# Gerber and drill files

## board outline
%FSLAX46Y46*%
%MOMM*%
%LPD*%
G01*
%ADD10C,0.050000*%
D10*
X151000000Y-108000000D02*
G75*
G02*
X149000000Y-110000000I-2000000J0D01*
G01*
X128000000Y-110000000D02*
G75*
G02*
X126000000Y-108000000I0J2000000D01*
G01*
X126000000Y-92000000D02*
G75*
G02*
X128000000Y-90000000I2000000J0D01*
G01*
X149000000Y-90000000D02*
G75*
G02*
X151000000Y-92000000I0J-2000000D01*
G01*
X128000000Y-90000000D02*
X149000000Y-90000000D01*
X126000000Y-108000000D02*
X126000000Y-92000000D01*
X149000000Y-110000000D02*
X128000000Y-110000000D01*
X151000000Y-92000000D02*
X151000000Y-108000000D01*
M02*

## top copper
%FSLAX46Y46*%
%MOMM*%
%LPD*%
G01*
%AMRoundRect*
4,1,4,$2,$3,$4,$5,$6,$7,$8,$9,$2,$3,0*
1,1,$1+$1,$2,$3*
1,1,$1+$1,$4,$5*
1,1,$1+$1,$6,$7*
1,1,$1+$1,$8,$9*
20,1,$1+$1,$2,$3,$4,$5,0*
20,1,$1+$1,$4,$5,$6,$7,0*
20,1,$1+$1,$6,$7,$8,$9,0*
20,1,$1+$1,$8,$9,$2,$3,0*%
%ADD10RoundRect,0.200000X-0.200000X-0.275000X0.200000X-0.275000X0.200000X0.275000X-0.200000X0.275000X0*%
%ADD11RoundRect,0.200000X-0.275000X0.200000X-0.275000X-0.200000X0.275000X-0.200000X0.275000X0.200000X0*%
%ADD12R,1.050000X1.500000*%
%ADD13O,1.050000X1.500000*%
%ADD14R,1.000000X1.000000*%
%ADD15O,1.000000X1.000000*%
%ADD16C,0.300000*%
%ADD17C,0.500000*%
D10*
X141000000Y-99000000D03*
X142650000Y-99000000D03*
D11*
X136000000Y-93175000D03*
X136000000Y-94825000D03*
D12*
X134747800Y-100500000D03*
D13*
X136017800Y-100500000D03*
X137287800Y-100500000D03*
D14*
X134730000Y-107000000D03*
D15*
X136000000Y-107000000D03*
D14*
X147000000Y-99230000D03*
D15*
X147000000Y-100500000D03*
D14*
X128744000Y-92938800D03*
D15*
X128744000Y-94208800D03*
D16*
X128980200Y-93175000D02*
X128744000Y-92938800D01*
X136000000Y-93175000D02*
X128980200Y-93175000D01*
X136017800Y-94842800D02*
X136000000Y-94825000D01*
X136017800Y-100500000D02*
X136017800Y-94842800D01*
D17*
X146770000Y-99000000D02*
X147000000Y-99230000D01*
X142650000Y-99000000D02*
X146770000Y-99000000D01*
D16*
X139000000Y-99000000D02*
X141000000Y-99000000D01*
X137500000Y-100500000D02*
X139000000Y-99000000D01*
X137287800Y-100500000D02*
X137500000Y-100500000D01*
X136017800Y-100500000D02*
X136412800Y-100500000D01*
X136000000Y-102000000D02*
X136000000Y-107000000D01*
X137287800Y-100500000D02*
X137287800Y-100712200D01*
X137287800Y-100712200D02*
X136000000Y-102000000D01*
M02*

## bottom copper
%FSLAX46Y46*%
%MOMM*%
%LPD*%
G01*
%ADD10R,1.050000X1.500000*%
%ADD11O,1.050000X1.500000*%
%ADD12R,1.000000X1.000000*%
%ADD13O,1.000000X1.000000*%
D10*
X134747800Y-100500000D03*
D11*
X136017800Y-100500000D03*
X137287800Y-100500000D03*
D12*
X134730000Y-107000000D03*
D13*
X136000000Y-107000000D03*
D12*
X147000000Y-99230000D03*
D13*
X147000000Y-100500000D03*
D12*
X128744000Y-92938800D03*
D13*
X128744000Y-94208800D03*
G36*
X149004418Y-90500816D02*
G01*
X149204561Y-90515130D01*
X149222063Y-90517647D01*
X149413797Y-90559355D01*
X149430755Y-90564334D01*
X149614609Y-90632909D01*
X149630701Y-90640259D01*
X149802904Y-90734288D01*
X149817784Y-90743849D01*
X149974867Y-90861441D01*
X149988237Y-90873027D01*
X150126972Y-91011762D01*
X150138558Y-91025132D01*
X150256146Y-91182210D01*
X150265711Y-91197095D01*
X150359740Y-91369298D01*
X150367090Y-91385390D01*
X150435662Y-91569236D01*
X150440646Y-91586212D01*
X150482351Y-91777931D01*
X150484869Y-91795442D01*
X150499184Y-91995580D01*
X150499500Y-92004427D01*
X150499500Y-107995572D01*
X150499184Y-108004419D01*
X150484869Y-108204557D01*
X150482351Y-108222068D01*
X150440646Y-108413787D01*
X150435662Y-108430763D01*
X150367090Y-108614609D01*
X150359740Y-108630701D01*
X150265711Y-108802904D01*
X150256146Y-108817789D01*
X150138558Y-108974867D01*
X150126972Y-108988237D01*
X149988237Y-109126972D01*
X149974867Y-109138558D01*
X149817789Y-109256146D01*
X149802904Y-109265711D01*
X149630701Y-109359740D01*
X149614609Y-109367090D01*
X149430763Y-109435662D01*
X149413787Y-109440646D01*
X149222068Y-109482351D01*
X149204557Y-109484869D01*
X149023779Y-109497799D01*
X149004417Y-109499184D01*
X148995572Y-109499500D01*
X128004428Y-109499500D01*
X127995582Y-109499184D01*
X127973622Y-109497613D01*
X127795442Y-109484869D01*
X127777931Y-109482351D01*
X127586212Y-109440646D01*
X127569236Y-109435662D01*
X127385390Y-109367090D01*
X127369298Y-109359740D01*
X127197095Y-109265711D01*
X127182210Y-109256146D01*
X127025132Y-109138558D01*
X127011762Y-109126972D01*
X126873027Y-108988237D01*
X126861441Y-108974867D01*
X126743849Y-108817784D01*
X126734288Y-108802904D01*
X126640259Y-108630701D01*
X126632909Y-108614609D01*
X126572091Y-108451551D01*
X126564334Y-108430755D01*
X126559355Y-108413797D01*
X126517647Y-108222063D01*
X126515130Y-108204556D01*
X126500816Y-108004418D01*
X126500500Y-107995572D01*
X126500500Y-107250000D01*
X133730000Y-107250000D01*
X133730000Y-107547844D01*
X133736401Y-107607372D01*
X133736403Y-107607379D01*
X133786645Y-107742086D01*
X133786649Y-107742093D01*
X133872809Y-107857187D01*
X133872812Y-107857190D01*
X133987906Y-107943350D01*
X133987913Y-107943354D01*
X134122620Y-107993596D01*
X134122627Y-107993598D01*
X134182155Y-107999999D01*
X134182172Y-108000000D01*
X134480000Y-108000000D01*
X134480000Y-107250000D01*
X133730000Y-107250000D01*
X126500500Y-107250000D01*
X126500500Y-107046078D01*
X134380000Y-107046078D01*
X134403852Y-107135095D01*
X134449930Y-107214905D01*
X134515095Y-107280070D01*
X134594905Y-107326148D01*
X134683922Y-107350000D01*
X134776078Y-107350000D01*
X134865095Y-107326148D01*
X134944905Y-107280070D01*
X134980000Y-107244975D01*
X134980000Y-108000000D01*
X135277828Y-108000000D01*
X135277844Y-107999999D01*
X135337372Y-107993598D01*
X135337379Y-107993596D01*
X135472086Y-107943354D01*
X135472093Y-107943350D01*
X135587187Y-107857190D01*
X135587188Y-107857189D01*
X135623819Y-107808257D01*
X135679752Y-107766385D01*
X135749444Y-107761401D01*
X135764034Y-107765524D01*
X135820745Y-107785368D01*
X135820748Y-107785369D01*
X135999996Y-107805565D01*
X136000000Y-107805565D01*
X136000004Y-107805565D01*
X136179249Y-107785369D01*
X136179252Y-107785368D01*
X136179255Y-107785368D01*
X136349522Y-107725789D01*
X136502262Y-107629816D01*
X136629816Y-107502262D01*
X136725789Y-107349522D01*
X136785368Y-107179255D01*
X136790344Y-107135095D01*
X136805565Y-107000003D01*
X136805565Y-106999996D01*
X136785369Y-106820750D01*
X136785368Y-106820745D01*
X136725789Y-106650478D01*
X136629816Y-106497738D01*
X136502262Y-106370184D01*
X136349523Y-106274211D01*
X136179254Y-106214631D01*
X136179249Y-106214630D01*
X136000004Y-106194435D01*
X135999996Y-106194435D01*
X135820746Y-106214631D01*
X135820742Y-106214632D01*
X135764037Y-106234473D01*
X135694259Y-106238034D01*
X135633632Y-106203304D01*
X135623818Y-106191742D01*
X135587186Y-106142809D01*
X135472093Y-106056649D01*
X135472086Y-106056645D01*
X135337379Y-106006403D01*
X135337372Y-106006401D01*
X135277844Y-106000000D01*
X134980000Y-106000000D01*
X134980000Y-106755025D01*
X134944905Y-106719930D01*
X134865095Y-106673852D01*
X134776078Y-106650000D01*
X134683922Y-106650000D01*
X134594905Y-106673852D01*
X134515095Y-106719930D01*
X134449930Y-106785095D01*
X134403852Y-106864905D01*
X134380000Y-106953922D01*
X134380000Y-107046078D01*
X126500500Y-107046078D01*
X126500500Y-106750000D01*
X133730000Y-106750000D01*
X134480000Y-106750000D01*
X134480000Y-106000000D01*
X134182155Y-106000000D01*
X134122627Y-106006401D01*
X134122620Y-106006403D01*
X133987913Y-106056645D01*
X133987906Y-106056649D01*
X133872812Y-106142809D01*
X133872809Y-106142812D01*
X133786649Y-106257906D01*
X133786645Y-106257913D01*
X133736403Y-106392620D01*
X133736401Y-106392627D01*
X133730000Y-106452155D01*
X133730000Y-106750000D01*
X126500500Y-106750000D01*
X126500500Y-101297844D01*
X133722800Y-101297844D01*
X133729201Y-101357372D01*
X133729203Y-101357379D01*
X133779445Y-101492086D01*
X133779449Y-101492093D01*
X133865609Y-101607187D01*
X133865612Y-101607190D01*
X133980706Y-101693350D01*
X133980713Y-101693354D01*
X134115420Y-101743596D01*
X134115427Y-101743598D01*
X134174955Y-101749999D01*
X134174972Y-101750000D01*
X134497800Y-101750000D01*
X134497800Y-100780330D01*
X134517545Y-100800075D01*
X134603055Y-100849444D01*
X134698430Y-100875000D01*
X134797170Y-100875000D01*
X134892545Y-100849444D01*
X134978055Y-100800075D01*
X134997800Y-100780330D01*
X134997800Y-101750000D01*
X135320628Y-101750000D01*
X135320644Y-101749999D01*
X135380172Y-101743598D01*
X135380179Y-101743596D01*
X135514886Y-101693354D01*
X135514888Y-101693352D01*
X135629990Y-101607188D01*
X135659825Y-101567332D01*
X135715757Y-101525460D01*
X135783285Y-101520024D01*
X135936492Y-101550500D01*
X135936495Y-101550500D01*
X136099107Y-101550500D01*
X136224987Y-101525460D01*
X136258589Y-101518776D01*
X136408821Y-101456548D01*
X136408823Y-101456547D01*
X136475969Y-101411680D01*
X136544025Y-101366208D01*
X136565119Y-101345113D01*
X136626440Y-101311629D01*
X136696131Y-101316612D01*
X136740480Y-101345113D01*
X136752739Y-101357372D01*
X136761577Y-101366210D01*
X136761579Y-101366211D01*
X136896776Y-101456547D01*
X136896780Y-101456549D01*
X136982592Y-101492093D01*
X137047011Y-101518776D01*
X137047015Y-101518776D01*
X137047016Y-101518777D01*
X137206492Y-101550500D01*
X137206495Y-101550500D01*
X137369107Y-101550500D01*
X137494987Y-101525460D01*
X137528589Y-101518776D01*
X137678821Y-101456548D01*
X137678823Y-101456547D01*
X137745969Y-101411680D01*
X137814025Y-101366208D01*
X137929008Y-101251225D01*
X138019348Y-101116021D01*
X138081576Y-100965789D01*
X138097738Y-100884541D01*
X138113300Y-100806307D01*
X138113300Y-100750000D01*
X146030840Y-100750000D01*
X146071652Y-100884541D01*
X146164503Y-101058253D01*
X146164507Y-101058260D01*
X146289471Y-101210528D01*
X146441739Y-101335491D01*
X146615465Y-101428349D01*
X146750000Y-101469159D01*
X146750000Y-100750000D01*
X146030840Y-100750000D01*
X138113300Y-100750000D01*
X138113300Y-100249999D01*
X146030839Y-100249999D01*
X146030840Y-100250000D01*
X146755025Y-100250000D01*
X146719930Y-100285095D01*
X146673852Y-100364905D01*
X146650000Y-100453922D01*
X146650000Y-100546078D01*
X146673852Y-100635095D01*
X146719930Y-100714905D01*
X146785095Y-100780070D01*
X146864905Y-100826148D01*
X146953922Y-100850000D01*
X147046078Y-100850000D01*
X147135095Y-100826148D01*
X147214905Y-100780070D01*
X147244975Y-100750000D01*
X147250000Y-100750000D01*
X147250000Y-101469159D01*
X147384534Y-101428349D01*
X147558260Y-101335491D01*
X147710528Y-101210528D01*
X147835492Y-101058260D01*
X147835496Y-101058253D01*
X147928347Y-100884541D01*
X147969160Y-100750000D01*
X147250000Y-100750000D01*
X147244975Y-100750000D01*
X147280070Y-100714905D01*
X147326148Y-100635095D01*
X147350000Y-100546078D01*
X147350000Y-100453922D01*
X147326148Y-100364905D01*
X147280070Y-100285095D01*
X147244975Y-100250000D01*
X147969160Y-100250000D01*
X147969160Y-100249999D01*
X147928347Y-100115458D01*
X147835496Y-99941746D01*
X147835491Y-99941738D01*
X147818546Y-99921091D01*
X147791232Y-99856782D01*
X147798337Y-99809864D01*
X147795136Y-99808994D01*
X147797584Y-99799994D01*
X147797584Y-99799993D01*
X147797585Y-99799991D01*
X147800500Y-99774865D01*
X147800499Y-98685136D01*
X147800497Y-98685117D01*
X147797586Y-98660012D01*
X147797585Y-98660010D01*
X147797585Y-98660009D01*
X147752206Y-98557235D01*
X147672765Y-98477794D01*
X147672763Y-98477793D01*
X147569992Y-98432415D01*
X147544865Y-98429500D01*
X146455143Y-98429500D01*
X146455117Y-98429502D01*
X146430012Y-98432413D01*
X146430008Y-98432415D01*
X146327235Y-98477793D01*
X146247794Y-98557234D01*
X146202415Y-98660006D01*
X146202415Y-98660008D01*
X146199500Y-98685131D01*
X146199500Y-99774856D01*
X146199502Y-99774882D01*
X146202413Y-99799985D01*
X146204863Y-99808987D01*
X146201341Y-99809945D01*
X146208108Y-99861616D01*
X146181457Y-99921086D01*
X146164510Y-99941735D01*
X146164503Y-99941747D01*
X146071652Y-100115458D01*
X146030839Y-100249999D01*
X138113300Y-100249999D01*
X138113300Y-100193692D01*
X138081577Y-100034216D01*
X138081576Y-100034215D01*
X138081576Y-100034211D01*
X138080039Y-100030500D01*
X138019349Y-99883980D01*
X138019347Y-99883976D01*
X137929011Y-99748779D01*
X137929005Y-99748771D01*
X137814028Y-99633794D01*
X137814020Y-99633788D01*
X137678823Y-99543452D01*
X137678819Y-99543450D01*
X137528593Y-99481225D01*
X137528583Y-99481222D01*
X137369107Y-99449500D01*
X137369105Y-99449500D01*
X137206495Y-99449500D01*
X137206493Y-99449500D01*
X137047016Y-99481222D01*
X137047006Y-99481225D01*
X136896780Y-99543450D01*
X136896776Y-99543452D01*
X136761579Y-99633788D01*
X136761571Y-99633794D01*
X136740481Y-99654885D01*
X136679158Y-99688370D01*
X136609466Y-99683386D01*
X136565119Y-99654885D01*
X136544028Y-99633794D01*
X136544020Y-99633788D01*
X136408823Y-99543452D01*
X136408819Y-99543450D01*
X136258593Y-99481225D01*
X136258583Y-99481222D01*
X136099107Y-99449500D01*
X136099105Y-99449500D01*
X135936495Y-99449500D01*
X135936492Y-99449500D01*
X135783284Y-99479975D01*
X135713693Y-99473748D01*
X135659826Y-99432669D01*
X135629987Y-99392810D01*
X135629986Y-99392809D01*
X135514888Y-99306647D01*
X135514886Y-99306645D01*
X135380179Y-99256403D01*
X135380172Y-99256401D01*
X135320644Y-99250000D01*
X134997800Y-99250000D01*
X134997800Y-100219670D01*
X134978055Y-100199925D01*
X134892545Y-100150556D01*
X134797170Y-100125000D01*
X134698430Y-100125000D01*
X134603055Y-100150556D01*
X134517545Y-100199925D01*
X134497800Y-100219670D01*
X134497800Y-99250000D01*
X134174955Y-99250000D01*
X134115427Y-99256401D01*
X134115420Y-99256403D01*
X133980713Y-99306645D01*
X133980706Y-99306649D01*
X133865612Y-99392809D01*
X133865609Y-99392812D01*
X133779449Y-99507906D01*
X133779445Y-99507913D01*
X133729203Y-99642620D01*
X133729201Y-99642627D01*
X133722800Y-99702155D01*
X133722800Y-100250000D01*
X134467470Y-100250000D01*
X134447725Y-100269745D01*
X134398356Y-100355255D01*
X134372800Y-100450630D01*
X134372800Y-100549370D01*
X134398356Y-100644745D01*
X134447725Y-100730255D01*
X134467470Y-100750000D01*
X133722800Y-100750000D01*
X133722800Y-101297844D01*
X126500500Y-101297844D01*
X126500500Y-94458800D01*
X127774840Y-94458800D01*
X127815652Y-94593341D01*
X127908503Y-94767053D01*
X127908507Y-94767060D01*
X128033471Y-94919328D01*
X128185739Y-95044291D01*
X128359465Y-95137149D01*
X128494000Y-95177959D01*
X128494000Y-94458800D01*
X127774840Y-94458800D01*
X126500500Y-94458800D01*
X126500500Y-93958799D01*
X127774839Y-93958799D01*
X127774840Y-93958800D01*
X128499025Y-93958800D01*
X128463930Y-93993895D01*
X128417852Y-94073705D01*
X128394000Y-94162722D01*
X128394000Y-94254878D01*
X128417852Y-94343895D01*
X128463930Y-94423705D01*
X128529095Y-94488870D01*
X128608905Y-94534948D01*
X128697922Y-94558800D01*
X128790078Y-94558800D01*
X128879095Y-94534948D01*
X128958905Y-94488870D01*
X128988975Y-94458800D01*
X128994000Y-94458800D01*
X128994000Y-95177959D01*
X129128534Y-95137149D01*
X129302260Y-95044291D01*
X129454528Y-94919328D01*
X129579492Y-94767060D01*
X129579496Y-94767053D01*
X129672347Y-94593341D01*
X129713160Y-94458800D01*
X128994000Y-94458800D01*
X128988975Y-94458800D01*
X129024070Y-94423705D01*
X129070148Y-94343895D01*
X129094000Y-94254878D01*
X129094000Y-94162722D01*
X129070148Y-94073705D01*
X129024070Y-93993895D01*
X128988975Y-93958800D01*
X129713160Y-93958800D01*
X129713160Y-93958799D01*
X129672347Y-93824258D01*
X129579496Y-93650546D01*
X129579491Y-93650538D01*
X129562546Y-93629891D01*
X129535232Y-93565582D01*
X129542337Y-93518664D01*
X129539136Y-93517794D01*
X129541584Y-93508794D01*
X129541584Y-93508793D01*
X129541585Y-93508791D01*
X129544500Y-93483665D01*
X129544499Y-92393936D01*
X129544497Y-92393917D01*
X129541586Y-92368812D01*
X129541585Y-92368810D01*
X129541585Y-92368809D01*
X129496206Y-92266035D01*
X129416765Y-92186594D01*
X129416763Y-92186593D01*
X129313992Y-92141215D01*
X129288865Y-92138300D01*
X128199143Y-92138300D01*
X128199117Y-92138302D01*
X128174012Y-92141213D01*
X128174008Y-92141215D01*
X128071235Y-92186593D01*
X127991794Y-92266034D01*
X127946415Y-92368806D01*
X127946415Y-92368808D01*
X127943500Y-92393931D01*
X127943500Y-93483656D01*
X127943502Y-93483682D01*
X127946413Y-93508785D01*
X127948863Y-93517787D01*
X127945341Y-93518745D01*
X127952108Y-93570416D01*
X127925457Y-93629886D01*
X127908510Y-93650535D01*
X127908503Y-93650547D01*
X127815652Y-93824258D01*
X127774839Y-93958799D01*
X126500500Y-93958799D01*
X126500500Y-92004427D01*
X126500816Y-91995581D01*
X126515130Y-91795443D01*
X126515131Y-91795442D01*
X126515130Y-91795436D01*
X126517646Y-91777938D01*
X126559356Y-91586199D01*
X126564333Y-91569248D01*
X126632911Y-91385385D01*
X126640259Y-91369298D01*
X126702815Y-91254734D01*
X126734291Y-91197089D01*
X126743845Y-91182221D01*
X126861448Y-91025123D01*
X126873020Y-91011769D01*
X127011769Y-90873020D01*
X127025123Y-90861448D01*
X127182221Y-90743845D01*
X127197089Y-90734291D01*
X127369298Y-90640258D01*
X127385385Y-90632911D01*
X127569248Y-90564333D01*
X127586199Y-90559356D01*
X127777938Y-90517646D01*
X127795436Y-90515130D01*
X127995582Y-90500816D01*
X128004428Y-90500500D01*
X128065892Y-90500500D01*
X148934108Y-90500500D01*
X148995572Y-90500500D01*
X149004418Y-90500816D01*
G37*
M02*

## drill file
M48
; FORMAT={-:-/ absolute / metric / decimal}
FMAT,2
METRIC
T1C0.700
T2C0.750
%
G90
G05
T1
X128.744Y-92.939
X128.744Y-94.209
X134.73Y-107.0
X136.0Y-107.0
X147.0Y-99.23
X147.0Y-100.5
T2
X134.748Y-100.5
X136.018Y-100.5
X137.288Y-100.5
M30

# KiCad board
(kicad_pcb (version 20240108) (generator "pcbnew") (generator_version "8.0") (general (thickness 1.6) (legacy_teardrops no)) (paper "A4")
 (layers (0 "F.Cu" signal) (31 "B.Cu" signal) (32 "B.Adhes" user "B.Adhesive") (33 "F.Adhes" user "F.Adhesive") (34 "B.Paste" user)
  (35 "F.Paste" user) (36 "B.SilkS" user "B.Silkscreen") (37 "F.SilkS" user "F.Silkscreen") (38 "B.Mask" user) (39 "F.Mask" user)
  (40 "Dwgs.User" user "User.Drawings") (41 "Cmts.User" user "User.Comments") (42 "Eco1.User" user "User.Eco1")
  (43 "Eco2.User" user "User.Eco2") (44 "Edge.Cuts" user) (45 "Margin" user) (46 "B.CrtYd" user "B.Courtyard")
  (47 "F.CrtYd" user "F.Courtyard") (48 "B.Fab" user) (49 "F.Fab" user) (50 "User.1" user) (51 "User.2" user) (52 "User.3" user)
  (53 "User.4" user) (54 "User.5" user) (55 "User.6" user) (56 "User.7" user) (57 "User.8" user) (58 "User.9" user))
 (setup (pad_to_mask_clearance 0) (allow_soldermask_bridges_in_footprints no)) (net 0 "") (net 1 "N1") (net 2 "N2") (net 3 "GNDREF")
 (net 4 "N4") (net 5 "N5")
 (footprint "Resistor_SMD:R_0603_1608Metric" (layer "F.Cu") (at 136 94 -90)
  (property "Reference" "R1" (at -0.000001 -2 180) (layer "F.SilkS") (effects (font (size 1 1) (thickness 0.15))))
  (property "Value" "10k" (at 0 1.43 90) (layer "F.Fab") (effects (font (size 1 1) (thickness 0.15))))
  (pad "1" smd roundrect (at -0.825 0 270) (size 0.8 0.95) (layers "F.Cu" "F.Paste" "F.Mask") (roundrect_rratio 0.25) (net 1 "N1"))
  (pad "2" smd roundrect (at 0.825 0 270) (size 0.8 0.95) (layers "F.Cu" "F.Paste" "F.Mask") (roundrect_rratio 0.25) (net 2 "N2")))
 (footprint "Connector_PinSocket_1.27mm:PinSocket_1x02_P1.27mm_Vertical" (layer "F.Cu") (at 134.73 107 90)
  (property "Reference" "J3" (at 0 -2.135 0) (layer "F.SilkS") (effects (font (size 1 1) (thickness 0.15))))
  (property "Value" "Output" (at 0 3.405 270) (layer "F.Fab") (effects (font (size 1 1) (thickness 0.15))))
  (pad "1" thru_hole rect (at 0 0 90) (size 1 1) (drill 0.7) (layers "*.Cu" "*.Mask") (remove_unused_layers no) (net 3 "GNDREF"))
  (pad "2" thru_hole oval (at 0 1.27 90) (size 1 1) (drill 0.7) (layers "*.Cu" "*.Mask") (remove_unused_layers no) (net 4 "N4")))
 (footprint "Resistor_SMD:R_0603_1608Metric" (layer "F.Cu") (at 141.825 99)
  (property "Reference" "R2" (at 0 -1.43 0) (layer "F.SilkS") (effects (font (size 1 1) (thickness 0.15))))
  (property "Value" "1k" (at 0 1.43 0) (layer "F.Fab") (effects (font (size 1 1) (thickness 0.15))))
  (pad "1" smd roundrect (at -0.825 0) (size 0.8 0.95) (layers "F.Cu" "F.Paste" "F.Mask") (roundrect_rratio 0.25) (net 4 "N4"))
  (pad "2" smd roundrect (at 0.825 0) (size 0.8 0.95) (layers "F.Cu" "F.Paste" "F.Mask") (roundrect_rratio 0.25) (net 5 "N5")))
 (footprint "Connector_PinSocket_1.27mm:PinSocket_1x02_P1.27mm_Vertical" (layer "F.Cu") (at 128.744 92.9388)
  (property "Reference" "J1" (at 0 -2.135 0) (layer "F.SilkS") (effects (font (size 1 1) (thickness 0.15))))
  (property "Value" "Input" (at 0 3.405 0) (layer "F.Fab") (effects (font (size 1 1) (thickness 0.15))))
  (pad "1" thru_hole rect (at 0 0) (size 1 1) (drill 0.7) (layers "*.Cu" "*.Mask") (remove_unused_layers no) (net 1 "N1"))
  (pad "2" thru_hole oval (at 0 1.27) (size 1 1) (drill 0.7) (layers "*.Cu" "*.Mask") (remove_unused_layers no) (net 3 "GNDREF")))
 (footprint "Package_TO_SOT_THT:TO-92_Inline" (layer "F.Cu") (at 134.7478 100.5)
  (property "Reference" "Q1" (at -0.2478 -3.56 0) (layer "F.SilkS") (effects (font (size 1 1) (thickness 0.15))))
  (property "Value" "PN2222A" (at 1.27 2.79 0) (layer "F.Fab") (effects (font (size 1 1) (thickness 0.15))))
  (pad "1" thru_hole rect (at 0 0) (size 1.05 1.5) (drill 0.75) (layers "*.Cu" "*.Mask") (remove_unused_layers no) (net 3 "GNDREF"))
  (pad "2" thru_hole oval (at 1.27 0) (size 1.05 1.5) (drill 0.75) (layers "*.Cu" "*.Mask") (remove_unused_layers no) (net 2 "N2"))
  (pad "3" thru_hole oval (at 2.54 0) (size 1.05 1.5) (drill 0.75) (layers "*.Cu" "*.Mask") (remove_unused_layers no) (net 4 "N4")))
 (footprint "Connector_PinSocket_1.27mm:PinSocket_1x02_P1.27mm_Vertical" (layer "F.Cu") (at 147 99.23)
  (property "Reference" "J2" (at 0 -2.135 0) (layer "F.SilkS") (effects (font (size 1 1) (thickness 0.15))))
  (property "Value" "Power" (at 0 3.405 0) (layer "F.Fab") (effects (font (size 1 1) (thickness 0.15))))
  (pad "1" thru_hole rect (at 0 0) (size 1 1) (drill 0.7) (layers "*.Cu" "*.Mask") (remove_unused_layers no) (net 5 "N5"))
  (pad "2" thru_hole oval (at 0 1.27) (size 1 1) (drill 0.7) (layers "*.Cu" "*.Mask") (remove_unused_layers no) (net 3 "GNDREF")))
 (gr_arc (start 149 90) (mid 150.414214 90.585786) (end 151 92) (stroke (width 0.05) (type default)) (layer "Edge.Cuts"))
 (gr_arc (start 128 110) (mid 126.585786 109.414214) (end 126 108) (stroke (width 0.05) (type default)) (layer "Edge.Cuts"))
 (gr_line (start 149 110) (end 128 110) (stroke (width 0.05) (type default)) (layer "Edge.Cuts"))
 (gr_line (start 151 92) (end 151 108) (stroke (width 0.05) (type default)) (layer "Edge.Cuts"))
 (gr_arc (start 126 92) (mid 126.585786 90.585786) (end 128 90) (stroke (width 0.05) (type default)) (layer "Edge.Cuts"))
 (gr_line (start 128 90) (end 149 90) (stroke (width 0.05) (type default)) (layer "Edge.Cuts"))
 (gr_line (start 126 108) (end 126 92) (stroke (width 0.05) (type default)) (layer "Edge.Cuts"))
 (gr_arc (start 151 108) (mid 150.414214 109.414214) (end 149 110) (stroke (width 0.05) (type default)) (layer "Edge.Cuts"))
 (segment (start 128.9802 93.175) (end 128.744 92.9388) (width 0.3) (layer "F.Cu") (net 1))
 (segment (start 136 93.175) (end 128.9802 93.175) (width 0.3) (layer "F.Cu") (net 1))
 (segment (start 142.65 99) (end 146.77 99) (width 0.5) (layer "F.Cu") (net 5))
 (segment (start 146.77 99) (end 147 99.23) (width 0.5) (layer "F.Cu") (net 5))
 (segment (start 137.2878 100.5) (end 137.5 100.5) (width 0.3) (layer "F.Cu") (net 4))
 (segment (start 139 99) (end 141 99) (width 0.3) (layer "F.Cu") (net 4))
 (segment (start 137.5 100.5) (end 139 99) (width 0.3) (layer "F.Cu") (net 4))
 (segment (start 136 102) (end 136 107) (width 0.3) (layer "F.Cu") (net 4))
 (segment (start 137.2878 100.7122) (end 136 102) (width 0.3) (layer "F.Cu") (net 4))
 (segment (start 137.2878 100.5) (end 137.2878 100.7122) (width 0.3) (layer "F.Cu") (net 4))
 (segment (start 136.0178 100.5) (end 136.0178 94.8428) (width 0.3) (layer "F.Cu") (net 2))
 (segment (start 136.0178 100.5) (end 136.4128 100.5) (width 0.3) (layer "F.Cu") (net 2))
 (segment (start 136.0178 94.8428) (end 136 94.825) (width 0.3) (layer "F.Cu") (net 2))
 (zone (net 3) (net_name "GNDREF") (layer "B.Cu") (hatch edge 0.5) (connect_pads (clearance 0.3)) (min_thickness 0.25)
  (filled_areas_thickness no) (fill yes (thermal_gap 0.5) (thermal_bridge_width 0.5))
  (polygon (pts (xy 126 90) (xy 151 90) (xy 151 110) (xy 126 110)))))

